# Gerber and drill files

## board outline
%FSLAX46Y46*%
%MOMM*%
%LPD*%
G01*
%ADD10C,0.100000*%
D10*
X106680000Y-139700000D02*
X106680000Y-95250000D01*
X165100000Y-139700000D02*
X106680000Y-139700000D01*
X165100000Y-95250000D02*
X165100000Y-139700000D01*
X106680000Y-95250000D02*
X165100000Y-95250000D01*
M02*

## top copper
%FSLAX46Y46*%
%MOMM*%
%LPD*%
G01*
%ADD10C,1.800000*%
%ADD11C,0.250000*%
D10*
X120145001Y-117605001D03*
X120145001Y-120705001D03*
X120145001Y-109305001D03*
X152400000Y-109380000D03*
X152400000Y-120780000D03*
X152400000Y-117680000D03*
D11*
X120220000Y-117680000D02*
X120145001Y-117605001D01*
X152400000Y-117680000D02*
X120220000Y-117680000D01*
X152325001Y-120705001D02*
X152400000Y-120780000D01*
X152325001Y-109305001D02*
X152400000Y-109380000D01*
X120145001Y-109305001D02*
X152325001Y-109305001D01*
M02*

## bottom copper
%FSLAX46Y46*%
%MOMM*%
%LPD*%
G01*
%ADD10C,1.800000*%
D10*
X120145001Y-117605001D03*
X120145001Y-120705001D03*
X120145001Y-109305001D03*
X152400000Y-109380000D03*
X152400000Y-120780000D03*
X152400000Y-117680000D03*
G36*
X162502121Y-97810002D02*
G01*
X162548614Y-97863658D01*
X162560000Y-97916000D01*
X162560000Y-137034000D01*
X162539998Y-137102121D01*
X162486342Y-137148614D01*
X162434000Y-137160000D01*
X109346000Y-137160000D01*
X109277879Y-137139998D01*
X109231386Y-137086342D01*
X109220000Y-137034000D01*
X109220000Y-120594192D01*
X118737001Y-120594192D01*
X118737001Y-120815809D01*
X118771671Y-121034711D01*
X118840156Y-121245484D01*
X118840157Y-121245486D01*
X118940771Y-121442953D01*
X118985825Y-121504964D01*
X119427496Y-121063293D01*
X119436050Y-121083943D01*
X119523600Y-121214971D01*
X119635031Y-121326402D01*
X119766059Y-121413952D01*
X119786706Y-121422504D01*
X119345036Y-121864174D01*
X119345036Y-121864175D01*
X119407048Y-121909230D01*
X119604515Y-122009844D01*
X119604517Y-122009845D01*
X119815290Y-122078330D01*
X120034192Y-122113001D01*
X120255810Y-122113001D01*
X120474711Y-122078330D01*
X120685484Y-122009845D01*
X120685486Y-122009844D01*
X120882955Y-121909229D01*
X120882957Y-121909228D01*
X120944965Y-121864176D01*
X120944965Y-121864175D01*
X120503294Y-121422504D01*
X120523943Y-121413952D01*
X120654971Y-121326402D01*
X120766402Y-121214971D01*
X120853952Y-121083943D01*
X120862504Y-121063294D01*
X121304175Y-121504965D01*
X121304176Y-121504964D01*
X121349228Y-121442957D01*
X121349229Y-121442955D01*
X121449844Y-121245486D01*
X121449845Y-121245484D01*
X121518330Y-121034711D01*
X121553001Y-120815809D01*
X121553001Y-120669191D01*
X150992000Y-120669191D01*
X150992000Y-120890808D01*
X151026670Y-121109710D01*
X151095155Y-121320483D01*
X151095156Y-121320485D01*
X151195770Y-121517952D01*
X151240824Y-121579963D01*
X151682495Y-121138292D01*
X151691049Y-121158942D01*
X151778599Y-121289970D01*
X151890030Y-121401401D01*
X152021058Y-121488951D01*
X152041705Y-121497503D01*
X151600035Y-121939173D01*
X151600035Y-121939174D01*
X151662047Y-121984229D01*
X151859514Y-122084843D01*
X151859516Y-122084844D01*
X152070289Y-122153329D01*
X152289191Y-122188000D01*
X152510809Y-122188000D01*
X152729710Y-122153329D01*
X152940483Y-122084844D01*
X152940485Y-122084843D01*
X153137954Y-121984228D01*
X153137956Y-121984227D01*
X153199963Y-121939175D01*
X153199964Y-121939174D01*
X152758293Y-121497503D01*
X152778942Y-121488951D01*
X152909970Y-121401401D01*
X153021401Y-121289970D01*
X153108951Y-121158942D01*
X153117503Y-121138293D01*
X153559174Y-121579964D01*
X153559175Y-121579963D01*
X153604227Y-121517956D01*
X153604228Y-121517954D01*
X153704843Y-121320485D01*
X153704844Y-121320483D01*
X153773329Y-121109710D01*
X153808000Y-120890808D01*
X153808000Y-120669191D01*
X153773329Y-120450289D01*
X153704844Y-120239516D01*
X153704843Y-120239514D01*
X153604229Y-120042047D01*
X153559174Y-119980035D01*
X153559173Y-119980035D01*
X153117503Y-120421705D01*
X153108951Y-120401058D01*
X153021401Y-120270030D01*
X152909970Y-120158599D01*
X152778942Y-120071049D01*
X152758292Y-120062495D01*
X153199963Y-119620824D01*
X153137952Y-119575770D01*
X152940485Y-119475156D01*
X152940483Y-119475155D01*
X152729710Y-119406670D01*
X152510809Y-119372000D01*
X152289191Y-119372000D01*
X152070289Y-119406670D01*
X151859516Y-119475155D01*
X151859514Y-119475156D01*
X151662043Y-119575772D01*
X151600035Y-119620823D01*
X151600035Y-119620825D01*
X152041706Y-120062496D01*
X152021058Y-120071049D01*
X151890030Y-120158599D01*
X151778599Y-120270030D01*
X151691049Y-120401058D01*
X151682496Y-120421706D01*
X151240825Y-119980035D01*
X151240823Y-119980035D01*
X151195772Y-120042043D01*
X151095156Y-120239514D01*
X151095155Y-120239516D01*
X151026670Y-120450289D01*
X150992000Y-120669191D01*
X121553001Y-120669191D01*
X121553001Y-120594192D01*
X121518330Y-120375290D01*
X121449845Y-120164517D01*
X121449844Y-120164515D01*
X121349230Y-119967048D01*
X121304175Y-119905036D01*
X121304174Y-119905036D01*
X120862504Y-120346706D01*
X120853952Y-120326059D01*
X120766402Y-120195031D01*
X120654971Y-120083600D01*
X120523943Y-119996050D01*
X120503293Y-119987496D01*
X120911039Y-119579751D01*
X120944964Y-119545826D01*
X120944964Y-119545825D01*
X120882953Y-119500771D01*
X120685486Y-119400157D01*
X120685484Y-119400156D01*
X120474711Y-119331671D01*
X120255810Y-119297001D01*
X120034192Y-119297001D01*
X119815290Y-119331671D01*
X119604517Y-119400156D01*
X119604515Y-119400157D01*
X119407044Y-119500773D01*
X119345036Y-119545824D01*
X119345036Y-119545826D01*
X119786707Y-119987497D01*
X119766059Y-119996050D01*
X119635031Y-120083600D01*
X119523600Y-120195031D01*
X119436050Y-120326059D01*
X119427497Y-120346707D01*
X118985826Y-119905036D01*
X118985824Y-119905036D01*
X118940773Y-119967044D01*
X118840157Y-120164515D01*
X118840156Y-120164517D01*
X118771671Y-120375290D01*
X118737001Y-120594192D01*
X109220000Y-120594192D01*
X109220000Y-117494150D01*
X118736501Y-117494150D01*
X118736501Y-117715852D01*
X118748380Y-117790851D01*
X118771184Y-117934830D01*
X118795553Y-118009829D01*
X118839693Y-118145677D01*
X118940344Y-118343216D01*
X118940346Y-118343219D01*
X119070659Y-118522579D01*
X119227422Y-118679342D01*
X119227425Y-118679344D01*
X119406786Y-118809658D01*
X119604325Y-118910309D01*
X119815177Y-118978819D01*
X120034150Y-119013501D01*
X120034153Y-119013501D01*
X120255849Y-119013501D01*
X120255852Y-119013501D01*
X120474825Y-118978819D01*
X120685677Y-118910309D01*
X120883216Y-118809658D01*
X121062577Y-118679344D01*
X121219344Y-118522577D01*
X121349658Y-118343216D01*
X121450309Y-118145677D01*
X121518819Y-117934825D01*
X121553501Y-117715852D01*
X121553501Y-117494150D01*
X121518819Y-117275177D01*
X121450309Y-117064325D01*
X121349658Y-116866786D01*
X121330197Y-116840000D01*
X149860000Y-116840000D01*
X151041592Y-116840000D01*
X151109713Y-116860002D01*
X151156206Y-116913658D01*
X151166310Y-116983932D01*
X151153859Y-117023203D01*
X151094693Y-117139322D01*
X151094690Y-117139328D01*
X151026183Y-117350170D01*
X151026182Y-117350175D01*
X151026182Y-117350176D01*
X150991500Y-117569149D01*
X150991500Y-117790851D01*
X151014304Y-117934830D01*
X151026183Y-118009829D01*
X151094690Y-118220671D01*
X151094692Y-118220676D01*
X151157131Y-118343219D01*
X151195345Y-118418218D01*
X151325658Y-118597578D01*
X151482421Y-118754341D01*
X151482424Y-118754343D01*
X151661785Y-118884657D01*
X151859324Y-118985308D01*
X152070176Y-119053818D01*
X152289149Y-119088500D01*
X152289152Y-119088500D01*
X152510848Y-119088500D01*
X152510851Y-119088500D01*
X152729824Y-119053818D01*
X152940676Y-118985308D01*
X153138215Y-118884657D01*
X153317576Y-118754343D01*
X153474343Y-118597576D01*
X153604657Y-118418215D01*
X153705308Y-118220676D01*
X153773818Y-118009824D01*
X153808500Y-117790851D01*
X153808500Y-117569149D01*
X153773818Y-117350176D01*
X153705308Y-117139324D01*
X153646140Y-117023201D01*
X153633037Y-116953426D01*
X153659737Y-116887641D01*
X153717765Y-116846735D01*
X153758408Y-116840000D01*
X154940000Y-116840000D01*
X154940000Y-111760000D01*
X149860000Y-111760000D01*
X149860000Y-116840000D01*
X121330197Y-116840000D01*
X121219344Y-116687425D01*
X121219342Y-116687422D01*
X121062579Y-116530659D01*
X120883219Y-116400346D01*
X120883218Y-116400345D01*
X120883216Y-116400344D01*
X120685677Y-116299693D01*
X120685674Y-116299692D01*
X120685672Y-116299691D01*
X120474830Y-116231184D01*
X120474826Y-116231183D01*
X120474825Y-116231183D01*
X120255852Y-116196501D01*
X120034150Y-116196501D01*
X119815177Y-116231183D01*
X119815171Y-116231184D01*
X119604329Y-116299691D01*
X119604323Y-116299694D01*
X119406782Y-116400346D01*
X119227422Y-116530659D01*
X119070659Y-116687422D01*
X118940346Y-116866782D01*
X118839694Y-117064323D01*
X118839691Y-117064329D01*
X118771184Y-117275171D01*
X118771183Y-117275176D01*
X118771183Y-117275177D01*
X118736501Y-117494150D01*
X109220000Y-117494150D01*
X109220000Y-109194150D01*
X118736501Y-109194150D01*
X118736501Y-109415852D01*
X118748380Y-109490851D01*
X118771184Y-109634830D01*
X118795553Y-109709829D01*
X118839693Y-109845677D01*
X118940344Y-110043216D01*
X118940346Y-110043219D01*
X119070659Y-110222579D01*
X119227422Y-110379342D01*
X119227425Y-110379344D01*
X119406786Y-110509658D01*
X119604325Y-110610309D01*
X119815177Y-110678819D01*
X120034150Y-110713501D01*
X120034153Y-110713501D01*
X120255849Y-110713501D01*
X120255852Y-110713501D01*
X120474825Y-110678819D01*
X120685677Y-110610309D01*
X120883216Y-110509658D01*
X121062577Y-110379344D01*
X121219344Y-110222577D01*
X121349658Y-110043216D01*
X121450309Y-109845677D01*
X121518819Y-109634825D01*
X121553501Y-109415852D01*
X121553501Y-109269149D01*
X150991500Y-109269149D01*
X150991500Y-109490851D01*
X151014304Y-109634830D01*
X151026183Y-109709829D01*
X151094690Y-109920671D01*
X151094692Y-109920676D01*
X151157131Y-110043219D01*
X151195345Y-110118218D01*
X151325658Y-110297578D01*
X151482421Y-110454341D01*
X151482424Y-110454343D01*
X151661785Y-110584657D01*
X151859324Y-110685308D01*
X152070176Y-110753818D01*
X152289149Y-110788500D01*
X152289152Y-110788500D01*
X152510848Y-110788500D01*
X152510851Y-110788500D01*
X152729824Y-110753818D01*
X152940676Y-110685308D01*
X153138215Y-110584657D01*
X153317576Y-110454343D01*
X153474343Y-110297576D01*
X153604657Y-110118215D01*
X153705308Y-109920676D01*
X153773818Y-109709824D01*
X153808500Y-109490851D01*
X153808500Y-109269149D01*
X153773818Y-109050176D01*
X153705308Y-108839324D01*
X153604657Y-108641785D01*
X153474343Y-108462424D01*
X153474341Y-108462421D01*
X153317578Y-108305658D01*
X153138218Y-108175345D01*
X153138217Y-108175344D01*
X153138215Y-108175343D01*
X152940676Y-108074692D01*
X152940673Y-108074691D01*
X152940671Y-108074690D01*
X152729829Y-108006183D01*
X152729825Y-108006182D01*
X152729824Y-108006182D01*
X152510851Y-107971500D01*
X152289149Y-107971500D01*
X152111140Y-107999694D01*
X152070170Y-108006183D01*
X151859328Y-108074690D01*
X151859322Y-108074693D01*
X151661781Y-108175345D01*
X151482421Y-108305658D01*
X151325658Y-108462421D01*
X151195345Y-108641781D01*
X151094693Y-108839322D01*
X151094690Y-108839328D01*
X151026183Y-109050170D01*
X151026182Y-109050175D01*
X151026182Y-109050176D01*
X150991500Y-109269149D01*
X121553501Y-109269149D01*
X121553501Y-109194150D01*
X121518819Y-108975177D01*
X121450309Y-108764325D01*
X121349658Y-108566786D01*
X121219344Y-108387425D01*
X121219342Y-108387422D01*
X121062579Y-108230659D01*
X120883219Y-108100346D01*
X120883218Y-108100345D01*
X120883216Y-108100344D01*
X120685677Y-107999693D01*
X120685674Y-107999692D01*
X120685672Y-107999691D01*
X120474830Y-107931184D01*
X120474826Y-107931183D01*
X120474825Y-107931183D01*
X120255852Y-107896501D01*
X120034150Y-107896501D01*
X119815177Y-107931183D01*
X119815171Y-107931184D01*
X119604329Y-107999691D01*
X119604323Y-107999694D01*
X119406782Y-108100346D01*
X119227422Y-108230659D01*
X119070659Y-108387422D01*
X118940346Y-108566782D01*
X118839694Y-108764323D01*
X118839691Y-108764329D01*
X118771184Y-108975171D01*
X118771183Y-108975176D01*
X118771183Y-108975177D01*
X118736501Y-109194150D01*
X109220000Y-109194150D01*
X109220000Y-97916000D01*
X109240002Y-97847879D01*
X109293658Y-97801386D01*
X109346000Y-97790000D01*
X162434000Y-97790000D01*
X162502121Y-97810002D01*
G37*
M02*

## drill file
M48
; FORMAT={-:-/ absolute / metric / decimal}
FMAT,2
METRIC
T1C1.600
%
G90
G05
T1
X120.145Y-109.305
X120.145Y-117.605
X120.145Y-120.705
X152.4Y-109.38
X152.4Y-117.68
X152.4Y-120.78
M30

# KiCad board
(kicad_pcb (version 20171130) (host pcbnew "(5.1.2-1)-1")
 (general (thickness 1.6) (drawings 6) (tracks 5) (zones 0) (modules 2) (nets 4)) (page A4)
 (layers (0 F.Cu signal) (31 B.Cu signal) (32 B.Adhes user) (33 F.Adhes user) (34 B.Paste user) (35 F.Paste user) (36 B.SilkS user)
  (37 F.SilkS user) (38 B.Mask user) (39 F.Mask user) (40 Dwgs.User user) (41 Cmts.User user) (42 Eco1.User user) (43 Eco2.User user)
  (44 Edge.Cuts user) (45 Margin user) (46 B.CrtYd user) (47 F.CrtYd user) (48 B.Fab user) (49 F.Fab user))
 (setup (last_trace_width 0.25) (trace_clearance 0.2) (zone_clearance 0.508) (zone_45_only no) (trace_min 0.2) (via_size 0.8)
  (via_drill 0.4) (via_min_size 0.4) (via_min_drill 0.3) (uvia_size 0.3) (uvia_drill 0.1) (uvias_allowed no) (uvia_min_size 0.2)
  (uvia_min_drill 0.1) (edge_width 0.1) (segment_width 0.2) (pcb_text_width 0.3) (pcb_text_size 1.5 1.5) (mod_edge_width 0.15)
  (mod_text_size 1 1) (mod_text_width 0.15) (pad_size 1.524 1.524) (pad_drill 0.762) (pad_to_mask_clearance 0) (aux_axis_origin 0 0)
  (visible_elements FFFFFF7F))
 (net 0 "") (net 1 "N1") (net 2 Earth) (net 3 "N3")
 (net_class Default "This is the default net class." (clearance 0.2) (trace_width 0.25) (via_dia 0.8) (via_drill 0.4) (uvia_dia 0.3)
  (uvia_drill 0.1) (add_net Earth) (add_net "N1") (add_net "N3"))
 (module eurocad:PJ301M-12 (layer F.Cu) (at 120.145001 114.225001)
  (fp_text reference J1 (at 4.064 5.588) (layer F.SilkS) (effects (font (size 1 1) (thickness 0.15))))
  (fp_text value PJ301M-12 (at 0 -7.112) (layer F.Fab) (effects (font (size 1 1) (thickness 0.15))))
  (pad 2 thru_hole circle (at 0 3.38) (size 1.8 1.8) (drill 1.6) (layers *.Cu *.Mask F.SilkS) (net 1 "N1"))
  (pad 1 thru_hole circle (at 0 6.48) (size 1.8 1.8) (drill 1.6) (layers *.Cu *.Mask F.SilkS) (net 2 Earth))
  (pad 3 thru_hole circle (at 0 -4.92) (size 1.8 1.8) (drill 1.6) (layers *.Cu *.Mask F.SilkS) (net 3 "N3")))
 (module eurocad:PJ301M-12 (layer F.Cu) (at 152.4 114.3)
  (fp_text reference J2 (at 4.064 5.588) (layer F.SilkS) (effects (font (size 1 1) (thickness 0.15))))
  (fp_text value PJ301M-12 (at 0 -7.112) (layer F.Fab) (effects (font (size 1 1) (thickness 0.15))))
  (pad 3 thru_hole circle (at 0 -4.92) (size 1.8 1.8) (drill 1.6) (layers *.Cu *.Mask F.SilkS) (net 3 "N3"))
  (pad 1 thru_hole circle (at 0 6.48) (size 1.8 1.8) (drill 1.6) (layers *.Cu *.Mask F.SilkS) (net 2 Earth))
  (pad 2 thru_hole circle (at 0 3.38) (size 1.8 1.8) (drill 1.6) (layers *.Cu *.Mask F.SilkS) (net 1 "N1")))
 (gr_line (start 106.68 139.7) (end 106.68 95.25) (layer Edge.Cuts) (width 0.1))
 (gr_line (start 165.1 139.7) (end 106.68 139.7) (layer Edge.Cuts) (width 0.1))
 (gr_line (start 165.1 95.25) (end 165.1 139.7) (layer Edge.Cuts) (width 0.1))
 (gr_line (start 106.68 95.25) (end 165.1 95.25) (layer Edge.Cuts) (width 0.1))
 (segment (start 120.22 117.68) (end 120.145001 117.605001) (width 0.25) (layer F.Cu) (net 1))
 (segment (start 152.4 117.68) (end 120.22 117.68) (width 0.25) (layer F.Cu) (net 1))
 (segment (start 152.325001 120.705001) (end 152.4 120.78) (width 0.25) (layer F.Cu) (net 2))
 (segment (start 152.325001 109.305001) (end 152.4 109.38) (width 0.25) (layer F.Cu) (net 3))
 (segment (start 120.145001 109.305001) (end 152.325001 109.305001) (width 0.25) (layer F.Cu) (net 3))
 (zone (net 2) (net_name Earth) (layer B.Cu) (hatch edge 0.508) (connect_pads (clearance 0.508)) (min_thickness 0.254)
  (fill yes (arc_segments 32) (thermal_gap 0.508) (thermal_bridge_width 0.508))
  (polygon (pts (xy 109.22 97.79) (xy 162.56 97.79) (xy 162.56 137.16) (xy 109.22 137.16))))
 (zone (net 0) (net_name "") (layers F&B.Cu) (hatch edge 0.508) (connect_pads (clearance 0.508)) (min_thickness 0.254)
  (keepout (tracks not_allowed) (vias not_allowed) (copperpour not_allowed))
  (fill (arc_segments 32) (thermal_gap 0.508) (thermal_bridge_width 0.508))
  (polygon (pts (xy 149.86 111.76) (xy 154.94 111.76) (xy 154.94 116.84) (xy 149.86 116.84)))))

